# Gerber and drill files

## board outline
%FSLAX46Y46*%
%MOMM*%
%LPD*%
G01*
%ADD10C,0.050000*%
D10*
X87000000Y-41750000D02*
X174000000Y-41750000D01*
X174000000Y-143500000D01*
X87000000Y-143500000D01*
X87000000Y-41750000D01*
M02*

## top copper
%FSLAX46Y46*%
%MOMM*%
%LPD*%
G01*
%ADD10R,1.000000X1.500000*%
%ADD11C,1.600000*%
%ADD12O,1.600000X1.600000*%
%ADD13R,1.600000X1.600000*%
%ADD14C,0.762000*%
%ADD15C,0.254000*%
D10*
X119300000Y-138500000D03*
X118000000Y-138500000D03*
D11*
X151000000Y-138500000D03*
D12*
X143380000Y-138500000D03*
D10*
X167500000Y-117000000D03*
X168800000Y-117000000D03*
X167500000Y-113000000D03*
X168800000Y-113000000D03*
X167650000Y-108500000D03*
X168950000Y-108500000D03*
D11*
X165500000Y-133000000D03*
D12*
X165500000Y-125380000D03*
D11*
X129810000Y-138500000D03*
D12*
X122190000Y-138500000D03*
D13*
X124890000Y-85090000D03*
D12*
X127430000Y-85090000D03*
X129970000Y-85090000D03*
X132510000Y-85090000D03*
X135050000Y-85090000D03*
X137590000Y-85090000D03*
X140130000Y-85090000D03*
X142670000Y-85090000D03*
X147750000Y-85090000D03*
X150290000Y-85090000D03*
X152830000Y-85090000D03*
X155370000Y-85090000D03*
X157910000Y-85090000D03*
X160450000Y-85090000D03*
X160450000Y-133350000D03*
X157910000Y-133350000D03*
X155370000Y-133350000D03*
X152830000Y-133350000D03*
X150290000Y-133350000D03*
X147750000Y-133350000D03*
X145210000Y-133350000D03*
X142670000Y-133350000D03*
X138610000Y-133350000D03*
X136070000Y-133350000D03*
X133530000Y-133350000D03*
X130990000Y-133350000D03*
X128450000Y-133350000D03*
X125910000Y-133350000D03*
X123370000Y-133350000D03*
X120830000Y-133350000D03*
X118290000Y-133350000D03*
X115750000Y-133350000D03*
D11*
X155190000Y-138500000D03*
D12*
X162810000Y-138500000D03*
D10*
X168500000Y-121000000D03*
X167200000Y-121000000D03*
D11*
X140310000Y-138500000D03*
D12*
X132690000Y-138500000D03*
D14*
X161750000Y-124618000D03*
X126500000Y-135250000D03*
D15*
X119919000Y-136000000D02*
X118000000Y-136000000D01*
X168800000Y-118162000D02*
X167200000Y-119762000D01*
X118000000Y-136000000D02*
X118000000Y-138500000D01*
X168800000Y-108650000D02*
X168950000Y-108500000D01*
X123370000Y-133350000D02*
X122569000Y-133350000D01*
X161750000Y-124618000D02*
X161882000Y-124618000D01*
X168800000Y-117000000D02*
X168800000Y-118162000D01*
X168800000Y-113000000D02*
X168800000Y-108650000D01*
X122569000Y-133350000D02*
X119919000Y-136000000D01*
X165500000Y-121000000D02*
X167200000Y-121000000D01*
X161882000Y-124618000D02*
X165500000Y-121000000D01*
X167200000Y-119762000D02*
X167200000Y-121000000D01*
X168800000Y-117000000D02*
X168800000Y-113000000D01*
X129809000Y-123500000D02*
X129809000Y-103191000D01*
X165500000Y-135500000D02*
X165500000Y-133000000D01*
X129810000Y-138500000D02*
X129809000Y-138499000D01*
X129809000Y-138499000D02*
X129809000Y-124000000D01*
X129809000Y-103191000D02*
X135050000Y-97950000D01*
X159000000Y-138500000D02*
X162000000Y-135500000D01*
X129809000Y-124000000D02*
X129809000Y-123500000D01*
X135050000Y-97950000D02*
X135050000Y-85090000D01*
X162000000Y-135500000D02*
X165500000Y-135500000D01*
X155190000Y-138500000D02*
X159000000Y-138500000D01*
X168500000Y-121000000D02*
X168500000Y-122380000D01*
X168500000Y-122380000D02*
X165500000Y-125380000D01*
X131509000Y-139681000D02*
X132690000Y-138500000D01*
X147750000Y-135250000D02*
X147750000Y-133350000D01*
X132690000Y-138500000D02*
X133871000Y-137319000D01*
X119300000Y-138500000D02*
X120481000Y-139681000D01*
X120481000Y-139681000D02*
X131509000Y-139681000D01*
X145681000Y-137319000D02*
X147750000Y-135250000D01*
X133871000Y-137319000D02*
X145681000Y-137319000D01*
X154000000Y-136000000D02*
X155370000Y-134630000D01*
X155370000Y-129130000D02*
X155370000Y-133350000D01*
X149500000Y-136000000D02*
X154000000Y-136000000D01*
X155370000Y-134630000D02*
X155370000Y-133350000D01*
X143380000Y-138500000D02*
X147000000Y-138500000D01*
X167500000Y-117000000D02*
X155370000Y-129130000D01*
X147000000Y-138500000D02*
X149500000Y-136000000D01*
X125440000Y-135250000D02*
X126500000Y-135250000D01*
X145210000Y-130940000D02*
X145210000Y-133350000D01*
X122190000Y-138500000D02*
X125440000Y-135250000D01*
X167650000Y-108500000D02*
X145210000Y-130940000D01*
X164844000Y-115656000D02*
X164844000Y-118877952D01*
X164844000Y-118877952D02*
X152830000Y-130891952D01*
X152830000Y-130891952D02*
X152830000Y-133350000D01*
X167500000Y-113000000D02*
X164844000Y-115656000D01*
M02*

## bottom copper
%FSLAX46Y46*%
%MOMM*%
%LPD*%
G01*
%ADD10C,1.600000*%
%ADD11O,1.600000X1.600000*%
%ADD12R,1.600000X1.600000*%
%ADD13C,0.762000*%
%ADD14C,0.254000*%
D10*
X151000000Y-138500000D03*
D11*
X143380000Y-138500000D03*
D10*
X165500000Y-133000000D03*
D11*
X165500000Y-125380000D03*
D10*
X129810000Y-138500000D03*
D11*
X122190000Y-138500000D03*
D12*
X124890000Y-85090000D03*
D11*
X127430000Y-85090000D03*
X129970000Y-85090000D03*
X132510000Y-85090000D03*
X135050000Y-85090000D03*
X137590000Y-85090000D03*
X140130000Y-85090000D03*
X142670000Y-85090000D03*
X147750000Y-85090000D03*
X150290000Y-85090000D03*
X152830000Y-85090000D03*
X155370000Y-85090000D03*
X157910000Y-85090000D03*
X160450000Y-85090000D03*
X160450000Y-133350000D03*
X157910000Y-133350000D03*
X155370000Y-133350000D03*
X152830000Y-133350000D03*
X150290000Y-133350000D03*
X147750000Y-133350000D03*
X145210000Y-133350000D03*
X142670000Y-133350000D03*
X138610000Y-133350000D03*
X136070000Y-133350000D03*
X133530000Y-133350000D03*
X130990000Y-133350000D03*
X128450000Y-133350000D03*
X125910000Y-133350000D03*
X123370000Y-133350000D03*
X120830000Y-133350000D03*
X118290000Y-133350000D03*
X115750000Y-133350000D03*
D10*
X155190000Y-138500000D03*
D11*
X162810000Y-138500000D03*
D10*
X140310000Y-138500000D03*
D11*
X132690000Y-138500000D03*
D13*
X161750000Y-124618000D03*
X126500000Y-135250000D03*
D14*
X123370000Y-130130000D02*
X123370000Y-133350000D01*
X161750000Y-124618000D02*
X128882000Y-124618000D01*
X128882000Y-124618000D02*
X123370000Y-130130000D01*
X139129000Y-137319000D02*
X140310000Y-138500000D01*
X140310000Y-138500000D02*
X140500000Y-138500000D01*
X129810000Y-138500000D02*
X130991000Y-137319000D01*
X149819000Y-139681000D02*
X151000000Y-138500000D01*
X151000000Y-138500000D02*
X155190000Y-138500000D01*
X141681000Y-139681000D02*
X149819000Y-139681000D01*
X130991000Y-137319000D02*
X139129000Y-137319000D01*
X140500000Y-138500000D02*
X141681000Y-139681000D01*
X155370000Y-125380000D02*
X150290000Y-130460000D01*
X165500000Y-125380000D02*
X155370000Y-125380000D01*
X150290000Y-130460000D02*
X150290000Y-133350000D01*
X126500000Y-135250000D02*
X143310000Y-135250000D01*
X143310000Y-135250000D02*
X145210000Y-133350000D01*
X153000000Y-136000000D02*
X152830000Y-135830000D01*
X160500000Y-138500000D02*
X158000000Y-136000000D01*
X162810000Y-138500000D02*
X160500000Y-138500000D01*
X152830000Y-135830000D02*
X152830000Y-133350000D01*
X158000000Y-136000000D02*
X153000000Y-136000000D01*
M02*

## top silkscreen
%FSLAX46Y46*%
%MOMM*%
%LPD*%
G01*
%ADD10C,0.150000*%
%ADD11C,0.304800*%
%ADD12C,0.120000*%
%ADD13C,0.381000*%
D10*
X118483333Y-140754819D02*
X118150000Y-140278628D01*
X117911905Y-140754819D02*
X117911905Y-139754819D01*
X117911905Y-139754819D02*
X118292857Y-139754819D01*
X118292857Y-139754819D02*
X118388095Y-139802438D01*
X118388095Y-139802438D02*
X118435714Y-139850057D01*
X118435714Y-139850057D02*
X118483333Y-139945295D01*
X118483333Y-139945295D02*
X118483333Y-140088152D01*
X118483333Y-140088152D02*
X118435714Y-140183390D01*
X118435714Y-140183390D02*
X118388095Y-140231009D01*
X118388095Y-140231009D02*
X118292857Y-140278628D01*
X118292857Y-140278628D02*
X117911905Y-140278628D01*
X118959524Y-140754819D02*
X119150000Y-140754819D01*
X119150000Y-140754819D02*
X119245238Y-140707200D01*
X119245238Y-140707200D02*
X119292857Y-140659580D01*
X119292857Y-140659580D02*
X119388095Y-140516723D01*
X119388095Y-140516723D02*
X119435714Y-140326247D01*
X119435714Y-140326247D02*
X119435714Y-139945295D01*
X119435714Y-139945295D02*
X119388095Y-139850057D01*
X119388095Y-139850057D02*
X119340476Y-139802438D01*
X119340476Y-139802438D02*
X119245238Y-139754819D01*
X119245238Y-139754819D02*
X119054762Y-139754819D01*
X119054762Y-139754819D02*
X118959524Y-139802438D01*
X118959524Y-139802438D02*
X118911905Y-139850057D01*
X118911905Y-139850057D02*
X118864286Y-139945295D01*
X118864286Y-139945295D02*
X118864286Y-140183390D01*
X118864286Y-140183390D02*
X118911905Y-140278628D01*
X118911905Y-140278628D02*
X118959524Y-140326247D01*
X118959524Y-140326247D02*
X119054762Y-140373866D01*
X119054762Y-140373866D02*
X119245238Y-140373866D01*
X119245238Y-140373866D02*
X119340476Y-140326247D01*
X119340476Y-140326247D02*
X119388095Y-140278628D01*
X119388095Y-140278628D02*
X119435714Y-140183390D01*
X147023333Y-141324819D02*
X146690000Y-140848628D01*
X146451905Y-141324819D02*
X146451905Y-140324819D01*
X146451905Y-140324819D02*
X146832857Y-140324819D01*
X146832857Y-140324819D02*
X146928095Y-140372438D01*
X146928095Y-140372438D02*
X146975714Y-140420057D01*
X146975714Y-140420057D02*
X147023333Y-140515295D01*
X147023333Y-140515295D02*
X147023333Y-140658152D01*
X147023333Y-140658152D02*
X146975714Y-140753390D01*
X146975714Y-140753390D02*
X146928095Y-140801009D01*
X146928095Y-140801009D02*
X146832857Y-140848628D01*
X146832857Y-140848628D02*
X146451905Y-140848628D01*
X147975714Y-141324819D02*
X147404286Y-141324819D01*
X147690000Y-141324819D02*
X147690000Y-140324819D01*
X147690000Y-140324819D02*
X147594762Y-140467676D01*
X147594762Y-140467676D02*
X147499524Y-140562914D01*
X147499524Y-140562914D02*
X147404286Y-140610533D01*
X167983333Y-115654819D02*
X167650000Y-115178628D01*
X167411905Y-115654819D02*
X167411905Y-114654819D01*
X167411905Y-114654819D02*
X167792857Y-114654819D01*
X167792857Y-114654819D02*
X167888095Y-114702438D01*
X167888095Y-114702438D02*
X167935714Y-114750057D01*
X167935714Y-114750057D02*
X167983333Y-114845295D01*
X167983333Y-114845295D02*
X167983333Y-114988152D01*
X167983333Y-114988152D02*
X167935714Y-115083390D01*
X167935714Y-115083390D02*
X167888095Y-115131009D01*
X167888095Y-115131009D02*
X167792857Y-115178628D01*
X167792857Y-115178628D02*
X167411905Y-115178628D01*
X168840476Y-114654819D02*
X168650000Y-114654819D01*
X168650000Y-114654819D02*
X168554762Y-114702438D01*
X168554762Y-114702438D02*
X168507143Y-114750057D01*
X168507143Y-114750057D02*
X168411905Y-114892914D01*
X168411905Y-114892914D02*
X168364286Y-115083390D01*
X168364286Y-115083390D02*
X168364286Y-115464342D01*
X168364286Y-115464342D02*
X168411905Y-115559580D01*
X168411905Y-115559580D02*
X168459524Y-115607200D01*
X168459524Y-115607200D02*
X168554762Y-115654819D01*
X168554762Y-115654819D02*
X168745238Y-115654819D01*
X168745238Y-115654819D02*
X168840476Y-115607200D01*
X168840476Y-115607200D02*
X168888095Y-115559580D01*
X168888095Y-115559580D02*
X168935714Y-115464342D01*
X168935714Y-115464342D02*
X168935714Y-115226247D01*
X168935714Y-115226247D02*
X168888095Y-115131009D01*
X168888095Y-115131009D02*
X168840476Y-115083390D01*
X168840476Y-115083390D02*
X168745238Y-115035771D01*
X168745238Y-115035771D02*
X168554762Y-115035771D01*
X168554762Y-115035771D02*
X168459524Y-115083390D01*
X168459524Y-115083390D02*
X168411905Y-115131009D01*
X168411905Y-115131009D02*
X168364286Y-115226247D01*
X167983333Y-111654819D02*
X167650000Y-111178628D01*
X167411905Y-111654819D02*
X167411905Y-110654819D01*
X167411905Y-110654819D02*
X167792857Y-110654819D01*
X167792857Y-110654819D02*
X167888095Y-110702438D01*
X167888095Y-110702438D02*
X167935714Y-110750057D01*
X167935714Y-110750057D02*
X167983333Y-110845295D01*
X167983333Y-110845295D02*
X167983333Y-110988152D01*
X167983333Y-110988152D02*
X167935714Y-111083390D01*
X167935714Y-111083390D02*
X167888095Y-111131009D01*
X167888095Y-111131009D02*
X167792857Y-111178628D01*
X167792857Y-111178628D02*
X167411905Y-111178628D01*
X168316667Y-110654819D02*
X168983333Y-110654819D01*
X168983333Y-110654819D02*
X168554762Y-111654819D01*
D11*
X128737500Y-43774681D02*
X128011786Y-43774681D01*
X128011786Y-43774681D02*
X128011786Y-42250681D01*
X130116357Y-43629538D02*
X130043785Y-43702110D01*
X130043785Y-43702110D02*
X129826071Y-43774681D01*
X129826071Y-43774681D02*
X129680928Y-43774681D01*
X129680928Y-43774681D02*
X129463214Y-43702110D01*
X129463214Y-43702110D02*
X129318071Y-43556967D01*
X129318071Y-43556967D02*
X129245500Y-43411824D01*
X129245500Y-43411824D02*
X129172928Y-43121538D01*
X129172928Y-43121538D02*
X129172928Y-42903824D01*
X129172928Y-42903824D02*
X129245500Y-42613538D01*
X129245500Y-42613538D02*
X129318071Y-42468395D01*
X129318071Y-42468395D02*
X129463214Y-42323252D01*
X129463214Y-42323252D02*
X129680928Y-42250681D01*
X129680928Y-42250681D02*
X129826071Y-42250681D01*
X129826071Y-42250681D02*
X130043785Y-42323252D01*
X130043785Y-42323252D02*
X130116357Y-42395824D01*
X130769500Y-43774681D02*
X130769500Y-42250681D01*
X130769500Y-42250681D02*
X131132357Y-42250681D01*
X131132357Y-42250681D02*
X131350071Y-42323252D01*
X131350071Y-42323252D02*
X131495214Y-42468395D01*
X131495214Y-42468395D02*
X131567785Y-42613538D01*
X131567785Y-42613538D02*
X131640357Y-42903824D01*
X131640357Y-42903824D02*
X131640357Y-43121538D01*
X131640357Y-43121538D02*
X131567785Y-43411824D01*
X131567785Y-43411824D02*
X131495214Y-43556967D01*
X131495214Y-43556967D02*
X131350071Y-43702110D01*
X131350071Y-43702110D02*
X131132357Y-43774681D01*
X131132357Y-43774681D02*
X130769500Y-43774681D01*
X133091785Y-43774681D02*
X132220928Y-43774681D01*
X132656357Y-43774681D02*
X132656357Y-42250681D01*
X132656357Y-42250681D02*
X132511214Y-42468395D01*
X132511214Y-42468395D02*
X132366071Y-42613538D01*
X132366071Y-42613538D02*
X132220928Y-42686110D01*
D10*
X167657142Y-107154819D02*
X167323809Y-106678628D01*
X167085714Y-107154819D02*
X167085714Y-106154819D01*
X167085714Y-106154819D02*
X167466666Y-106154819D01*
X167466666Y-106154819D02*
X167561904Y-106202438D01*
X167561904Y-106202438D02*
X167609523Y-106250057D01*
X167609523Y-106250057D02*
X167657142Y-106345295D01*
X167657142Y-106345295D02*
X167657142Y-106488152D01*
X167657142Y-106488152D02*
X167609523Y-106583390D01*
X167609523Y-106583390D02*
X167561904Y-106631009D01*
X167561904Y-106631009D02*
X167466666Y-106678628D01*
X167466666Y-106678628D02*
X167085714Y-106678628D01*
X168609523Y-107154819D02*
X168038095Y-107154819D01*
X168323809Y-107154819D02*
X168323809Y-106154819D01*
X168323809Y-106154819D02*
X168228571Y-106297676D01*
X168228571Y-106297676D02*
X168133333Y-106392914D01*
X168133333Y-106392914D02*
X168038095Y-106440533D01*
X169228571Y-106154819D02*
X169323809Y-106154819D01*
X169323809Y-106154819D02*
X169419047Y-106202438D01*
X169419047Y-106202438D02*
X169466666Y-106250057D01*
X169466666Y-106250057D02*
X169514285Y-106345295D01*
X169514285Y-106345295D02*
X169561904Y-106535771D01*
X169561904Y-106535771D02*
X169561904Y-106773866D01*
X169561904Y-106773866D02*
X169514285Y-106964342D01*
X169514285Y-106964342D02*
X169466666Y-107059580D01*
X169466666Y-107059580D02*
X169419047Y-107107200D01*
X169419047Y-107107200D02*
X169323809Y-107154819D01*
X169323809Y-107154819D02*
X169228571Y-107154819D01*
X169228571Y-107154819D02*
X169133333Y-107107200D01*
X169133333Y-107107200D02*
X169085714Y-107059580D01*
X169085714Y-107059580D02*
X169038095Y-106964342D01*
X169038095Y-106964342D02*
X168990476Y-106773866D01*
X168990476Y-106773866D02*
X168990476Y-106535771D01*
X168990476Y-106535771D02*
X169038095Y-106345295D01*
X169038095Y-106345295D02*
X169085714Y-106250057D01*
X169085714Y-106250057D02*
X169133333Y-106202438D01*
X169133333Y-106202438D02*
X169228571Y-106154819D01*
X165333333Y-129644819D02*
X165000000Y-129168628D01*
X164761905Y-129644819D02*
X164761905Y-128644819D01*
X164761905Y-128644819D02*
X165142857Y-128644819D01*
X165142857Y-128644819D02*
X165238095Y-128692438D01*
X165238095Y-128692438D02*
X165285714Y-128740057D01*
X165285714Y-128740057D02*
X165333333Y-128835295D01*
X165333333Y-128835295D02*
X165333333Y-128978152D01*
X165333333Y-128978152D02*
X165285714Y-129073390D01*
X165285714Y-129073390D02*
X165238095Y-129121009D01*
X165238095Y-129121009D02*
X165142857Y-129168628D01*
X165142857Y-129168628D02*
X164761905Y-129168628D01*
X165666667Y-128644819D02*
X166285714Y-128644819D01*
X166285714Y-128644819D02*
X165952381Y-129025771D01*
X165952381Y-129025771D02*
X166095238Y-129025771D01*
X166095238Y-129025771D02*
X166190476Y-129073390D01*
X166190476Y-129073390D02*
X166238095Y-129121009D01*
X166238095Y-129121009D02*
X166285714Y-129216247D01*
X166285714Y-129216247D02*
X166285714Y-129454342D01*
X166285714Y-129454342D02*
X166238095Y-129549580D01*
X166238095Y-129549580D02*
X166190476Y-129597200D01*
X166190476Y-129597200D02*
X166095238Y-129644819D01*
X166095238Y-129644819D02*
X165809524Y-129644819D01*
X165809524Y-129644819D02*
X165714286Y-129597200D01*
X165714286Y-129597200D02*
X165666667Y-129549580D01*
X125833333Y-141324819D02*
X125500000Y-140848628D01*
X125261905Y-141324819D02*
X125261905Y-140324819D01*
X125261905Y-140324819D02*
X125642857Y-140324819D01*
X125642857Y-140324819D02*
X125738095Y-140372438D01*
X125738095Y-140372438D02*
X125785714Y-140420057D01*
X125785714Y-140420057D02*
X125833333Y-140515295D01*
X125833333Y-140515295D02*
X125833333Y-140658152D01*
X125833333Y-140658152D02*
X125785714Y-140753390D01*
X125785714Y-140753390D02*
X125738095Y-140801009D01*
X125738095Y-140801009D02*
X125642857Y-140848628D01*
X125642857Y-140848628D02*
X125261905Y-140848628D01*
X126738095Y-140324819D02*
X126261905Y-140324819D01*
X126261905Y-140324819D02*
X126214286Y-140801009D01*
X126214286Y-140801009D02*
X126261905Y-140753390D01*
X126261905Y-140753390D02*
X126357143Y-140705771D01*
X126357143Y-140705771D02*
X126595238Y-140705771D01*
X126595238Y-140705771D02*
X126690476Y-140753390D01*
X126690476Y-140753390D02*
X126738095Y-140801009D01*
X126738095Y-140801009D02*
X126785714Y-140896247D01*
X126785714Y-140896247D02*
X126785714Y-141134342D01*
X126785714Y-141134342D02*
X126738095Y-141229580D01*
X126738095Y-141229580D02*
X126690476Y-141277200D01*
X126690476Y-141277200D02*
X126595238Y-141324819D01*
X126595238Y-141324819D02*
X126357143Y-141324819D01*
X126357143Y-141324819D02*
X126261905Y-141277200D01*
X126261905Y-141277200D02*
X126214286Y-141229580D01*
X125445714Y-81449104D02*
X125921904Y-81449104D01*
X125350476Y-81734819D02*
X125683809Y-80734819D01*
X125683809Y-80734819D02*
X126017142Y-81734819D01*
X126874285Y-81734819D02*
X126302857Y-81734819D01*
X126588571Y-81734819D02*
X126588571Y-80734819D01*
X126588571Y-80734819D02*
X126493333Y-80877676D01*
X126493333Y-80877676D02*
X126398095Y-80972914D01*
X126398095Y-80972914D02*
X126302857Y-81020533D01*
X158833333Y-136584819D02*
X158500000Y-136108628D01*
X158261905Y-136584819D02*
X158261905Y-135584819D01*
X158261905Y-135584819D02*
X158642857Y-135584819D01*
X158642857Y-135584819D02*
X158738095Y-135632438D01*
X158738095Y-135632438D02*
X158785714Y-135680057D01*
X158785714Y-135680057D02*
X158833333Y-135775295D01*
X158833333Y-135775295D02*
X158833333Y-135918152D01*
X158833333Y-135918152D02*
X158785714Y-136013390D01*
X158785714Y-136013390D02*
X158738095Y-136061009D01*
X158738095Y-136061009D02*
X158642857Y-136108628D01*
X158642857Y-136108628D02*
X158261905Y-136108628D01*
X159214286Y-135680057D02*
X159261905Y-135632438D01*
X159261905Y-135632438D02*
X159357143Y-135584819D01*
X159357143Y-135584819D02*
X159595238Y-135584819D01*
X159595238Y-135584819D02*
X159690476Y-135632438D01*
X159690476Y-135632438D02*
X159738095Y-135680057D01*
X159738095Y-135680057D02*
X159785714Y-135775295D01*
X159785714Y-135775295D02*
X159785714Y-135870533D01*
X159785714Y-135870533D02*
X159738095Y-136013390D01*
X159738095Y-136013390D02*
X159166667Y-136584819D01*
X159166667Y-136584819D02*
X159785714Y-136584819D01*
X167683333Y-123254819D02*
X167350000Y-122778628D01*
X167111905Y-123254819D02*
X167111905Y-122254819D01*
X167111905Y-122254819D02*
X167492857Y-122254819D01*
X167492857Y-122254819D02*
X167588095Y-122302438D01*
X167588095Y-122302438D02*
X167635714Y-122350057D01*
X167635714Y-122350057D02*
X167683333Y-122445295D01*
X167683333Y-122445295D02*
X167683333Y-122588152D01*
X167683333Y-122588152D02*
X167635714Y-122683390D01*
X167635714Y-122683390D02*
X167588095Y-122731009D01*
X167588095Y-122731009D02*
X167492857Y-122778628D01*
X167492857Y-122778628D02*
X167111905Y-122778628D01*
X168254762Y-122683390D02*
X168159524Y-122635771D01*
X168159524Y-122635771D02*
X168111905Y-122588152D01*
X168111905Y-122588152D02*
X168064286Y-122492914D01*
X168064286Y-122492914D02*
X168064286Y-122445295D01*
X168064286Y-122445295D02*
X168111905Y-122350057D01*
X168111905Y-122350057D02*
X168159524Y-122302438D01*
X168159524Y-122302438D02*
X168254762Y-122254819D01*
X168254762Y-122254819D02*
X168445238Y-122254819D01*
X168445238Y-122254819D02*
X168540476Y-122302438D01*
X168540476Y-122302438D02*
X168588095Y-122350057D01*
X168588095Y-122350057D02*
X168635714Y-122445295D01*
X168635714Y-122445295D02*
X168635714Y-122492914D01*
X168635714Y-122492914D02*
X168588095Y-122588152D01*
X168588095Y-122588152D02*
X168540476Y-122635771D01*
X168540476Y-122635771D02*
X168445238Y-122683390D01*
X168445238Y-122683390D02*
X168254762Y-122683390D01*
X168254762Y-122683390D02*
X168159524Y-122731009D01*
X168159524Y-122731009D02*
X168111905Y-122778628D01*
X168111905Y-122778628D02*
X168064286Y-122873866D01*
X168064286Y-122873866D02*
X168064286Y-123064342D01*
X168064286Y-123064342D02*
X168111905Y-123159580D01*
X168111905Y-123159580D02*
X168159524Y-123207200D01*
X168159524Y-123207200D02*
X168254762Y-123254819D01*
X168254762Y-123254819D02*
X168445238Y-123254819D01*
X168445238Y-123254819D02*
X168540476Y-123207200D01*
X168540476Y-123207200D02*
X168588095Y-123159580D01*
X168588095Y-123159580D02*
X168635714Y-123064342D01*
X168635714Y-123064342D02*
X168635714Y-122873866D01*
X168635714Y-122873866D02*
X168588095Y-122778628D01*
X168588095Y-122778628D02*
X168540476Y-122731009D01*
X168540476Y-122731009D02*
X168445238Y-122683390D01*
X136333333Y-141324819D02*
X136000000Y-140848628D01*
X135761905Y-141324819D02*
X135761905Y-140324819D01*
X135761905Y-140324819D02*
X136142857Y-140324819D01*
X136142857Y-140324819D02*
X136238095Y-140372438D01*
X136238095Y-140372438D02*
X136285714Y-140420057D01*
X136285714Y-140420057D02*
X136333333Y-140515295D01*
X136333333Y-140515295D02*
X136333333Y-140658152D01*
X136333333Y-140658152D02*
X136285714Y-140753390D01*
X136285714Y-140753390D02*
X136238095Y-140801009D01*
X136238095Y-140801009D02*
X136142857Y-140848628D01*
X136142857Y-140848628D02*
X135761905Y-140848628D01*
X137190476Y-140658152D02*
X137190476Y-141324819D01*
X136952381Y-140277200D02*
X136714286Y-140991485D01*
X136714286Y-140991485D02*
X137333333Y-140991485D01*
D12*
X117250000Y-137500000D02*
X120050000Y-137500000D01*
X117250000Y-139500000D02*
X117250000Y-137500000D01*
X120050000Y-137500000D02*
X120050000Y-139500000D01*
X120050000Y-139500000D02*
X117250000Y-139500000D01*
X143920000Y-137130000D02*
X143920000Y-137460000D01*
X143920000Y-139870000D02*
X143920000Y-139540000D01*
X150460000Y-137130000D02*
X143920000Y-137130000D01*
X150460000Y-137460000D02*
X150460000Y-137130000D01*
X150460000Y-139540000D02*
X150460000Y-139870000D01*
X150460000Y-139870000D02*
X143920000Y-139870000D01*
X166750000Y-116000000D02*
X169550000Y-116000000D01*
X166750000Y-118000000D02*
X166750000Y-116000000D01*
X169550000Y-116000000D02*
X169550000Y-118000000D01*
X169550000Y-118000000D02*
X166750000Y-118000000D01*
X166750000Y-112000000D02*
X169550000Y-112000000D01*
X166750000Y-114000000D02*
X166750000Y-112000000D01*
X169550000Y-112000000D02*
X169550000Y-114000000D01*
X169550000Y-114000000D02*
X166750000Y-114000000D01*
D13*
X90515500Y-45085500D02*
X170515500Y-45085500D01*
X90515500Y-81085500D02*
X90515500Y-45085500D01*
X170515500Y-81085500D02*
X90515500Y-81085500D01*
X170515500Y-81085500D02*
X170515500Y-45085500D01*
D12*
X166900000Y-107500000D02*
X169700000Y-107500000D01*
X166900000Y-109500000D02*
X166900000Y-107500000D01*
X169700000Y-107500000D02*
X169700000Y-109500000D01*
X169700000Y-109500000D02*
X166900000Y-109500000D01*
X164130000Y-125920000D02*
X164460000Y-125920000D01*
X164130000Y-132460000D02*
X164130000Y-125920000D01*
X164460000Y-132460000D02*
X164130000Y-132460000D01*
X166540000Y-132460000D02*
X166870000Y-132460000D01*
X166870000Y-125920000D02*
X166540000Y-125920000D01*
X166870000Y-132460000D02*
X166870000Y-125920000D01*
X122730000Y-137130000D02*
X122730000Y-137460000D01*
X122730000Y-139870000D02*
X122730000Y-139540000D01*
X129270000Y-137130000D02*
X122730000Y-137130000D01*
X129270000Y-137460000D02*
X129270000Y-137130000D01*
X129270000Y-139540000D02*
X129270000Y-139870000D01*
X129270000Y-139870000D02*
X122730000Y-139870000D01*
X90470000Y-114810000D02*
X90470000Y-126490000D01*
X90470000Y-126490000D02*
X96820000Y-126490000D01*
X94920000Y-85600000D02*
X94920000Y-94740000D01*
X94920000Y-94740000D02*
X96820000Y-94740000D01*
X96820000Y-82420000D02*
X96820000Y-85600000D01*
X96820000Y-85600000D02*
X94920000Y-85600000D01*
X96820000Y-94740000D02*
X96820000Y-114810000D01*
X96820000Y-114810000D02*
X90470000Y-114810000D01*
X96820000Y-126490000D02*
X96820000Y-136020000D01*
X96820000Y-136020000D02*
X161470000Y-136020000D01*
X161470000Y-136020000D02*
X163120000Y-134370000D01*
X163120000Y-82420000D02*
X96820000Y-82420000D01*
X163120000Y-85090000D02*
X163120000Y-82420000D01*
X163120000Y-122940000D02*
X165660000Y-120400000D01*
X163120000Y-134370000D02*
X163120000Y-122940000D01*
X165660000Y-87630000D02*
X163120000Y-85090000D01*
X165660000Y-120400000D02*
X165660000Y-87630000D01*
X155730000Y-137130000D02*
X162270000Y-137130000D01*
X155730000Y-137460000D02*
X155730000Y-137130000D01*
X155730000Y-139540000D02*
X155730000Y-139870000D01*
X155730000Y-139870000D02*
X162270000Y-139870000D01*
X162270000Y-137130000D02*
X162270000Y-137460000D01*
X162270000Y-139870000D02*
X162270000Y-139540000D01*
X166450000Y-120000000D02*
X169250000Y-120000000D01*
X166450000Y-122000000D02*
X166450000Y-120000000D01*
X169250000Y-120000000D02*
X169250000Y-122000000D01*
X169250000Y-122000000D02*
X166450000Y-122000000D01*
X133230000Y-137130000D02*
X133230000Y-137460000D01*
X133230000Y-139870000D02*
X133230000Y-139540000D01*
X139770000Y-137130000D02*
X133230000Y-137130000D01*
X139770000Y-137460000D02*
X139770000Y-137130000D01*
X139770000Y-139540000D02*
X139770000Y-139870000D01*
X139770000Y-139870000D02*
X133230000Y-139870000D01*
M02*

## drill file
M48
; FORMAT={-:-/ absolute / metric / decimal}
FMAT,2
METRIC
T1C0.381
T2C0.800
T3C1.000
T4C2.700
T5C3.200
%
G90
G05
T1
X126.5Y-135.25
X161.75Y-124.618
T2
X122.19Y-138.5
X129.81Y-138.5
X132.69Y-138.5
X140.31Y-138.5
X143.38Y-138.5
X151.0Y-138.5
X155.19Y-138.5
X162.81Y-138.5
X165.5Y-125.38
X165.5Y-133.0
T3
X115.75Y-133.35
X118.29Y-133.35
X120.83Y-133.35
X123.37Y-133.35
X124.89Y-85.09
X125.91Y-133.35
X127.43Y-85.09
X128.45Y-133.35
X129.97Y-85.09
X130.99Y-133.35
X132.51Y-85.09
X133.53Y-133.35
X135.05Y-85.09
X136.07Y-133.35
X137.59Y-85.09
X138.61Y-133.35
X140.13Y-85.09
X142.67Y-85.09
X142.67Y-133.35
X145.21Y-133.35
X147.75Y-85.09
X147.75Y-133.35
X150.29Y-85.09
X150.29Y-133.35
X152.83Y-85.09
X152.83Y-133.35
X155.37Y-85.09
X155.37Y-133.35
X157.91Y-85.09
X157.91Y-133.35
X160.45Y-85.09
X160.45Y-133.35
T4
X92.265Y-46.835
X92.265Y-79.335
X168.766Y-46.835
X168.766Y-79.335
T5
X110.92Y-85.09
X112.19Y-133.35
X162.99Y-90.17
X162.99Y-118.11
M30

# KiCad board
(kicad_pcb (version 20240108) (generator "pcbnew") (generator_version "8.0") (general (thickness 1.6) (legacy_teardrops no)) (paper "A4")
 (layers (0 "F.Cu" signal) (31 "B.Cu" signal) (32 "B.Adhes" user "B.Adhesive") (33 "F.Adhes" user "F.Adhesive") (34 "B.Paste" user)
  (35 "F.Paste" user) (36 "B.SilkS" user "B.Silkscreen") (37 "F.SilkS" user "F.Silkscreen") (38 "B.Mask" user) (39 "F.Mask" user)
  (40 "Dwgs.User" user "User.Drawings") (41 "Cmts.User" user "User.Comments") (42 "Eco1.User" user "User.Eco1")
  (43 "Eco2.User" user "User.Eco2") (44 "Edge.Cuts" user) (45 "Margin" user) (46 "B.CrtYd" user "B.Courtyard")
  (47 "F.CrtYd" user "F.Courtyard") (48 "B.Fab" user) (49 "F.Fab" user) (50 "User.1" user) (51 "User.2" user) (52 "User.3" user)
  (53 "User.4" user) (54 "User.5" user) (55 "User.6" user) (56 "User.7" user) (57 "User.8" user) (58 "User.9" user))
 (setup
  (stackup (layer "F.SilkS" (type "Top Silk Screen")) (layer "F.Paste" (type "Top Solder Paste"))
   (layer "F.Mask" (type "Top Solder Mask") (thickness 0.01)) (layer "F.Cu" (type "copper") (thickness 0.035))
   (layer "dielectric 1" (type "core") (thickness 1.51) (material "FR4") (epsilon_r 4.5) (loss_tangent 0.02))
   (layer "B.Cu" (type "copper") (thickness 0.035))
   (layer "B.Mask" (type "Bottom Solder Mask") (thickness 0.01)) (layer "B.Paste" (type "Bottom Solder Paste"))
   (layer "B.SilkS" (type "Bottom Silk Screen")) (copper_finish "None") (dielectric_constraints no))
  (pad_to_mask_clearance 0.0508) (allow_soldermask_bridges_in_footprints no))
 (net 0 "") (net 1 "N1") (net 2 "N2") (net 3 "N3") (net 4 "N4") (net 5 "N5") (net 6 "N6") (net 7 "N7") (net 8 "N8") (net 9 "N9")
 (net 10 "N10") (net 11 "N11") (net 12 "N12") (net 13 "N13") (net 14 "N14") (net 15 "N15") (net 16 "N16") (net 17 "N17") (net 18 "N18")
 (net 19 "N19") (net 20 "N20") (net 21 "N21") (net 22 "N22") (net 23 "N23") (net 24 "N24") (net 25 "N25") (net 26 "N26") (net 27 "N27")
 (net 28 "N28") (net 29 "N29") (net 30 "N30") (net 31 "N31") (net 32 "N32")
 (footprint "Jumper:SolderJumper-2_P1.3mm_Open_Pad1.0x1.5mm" (layer "F.Cu") (at 118.65 138.5 180)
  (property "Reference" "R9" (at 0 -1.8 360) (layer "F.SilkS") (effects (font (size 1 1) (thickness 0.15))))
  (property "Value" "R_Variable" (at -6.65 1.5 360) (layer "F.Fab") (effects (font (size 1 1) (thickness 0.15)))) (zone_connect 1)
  (fp_line (start 1.4 1) (end -1.4 1) (stroke (width 0.12) (type solid)) (layer "F.SilkS"))
  (fp_line (start 1.4 -1) (end 1.4 1) (stroke (width 0.12) (type solid)) (layer "F.SilkS"))
  (fp_line (start -1.4 1) (end -1.4 -1) (stroke (width 0.12) (type solid)) (layer "F.SilkS"))
  (fp_line (start -1.4 -1) (end 1.4 -1) (stroke (width 0.12) (type solid)) (layer "F.SilkS"))
  (pad "1" smd rect (at -0.65 0 180) (size 1 1.5) (layers "F.Cu" "F.Mask") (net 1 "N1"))
  (pad "2" smd rect (at 0.65 0 180) (size 1 1.5) (layers "F.Cu" "F.Mask") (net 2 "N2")))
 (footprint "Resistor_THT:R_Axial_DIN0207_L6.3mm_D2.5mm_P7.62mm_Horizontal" (layer "F.Cu") (at 151 138.5 180)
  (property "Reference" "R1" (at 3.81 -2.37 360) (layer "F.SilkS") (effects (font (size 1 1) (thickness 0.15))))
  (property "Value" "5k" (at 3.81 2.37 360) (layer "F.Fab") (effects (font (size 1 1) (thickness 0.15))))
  (fp_line (start 7.08 1.37) (end 7.08 1.04) (stroke (width 0.12) (type solid)) (layer "F.SilkS"))
  (fp_line (start 7.08 -1.37) (end 7.08 -1.04) (stroke (width 0.12) (type solid)) (layer "F.SilkS"))
  (fp_line (start 0.54 1.37) (end 7.08 1.37) (stroke (width 0.12) (type solid)) (layer "F.SilkS"))
  (fp_line (start 0.54 1.04) (end 0.54 1.37) (stroke (width 0.12) (type solid)) (layer "F.SilkS"))
  (fp_line (start 0.54 -1.04) (end 0.54 -1.37) (stroke (width 0.12) (type solid)) (layer "F.SilkS"))
  (fp_line (start 0.54 -1.37) (end 7.08 -1.37) (stroke (width 0.12) (type solid)) (layer "F.SilkS"))
  (pad "1" thru_hole circle (at 0 0 180) (size 1.6 1.6) (drill 0.8) (layers "*.Cu" "*.Mask") (remove_unused_layers no) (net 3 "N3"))
  (pad "2" thru_hole oval (at 7.62 0 180) (size 1.6 1.6) (drill 0.8) (layers "*.Cu" "*.Mask") (remove_unused_layers no) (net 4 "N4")))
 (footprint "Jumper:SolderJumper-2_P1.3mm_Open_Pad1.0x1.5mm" (layer "F.Cu") (at 168.15 117)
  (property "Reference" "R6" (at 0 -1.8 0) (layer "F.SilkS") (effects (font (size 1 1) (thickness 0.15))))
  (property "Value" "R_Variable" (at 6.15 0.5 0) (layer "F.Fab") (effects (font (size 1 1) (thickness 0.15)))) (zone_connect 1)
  (fp_line (start -1.4 -1) (end 1.4 -1) (stroke (width 0.12) (type solid)) (layer "F.SilkS"))
  (fp_line (start -1.4 1) (end -1.4 -1) (stroke (width 0.12) (type solid)) (layer "F.SilkS"))
  (fp_line (start 1.4 -1) (end 1.4 1) (stroke (width 0.12) (type solid)) (layer "F.SilkS"))
  (fp_line (start 1.4 1) (end -1.4 1) (stroke (width 0.12) (type solid)) (layer "F.SilkS"))
  (pad "1" smd rect (at -0.65 0) (size 1 1.5) (layers "F.Cu" "F.Mask") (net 4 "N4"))
  (pad "2" smd rect (at 0.65 0) (size 1 1.5) (layers "F.Cu" "F.Mask") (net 2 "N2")))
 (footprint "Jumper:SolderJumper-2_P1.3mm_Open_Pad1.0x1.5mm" (layer "F.Cu") (at 168.15 113)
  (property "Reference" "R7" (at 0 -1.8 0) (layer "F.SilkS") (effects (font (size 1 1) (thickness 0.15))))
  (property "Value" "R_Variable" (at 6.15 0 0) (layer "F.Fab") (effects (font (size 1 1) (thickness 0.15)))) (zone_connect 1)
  (fp_line (start -1.4 -1) (end 1.4 -1) (stroke (width 0.12) (type solid)) (layer "F.SilkS"))
  (fp_line (start -1.4 1) (end -1.4 -1) (stroke (width 0.12) (type solid)) (layer "F.SilkS"))
  (fp_line (start 1.4 -1) (end 1.4 1) (stroke (width 0.12) (type solid)) (layer "F.SilkS"))
  (fp_line (start 1.4 1) (end -1.4 1) (stroke (width 0.12) (type solid)) (layer "F.SilkS"))
  (pad "1" smd rect (at -0.65 0) (size 1 1.5) (layers "F.Cu" "F.Mask") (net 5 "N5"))
  (pad "2" smd rect (at 0.65 0) (size 1 1.5) (layers "F.Cu" "F.Mask") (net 2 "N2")))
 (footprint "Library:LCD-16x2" (layer "F.Cu") (at 130.5155 63.0855)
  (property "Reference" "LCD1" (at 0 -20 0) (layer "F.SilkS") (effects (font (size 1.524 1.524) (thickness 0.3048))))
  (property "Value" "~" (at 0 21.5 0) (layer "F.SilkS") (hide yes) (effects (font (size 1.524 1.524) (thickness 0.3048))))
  (fp_line (start -40 -18) (end 40 -18) (stroke (width 0.381) (type solid)) (layer "F.SilkS"))
  (fp_line (start -40 18) (end -40 -18) (stroke (width 0.381) (type solid)) (layer "F.SilkS"))
  (fp_line (start 40 18) (end -40 18) (stroke (width 0.381) (type solid)) (layer "F.SilkS"))
  (fp_line (start 40 18) (end 40 -18) (stroke (width 0.381) (type solid)) (layer "F.SilkS"))
  (pad "" np_thru_hole circle (at -38.25 -16.25) (size 0.01 0.01) (drill 2.7) (layers "F&B.Cu" "*.Mask"))
  (pad "" np_thru_hole circle (at -38.25 16.25 90) (size 0.01 0.01) (drill 2.7) (layers "F&B.Cu" "*.Mask"))
  (pad "" np_thru_hole circle (at 38.25 -16.25) (size 0.01 0.01) (drill 2.7) (layers "F&B.Cu" "*.Mask"))
  (pad "" np_thru_hole circle (at 38.25 16.25) (size 0.01 0.01) (drill 2.7) (layers "F&B.Cu" "*.Mask")))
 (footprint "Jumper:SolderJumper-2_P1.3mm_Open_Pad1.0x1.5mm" (layer "F.Cu") (at 168.3 108.5)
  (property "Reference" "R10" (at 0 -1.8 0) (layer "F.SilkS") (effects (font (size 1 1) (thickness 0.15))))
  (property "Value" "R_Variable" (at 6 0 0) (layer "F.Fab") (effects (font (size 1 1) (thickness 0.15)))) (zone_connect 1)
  (fp_line (start -1.4 -1) (end 1.4 -1) (stroke (width 0.12) (type solid)) (layer "F.SilkS"))
  (fp_line (start -1.4 1) (end -1.4 -1) (stroke (width 0.12) (type solid)) (layer "F.SilkS"))
  (fp_line (start 1.4 -1) (end 1.4 1) (stroke (width 0.12) (type solid)) (layer "F.SilkS"))
  (fp_line (start 1.4 1) (end -1.4 1) (stroke (width 0.12) (type solid)) (layer "F.SilkS"))
  (pad "1" smd rect (at -0.65 0) (size 1 1.5) (layers "F.Cu" "F.Mask") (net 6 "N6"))
  (pad "2" smd rect (at 0.65 0) (size 1 1.5) (layers "F.Cu" "F.Mask") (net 2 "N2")))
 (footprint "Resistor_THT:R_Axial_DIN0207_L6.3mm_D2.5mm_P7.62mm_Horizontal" (layer "F.Cu") (at 165.5 133 90)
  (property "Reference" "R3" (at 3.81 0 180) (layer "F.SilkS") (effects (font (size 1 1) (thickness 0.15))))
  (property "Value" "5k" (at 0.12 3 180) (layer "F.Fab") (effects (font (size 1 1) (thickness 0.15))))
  (fp_line (start 7.08 -1.37) (end 7.08 -1.04) (stroke (width 0.12) (type solid)) (layer "F.SilkS"))
  (fp_line (start 0.54 -1.37) (end 7.08 -1.37) (stroke (width 0.12) (type solid)) (layer "F.SilkS"))
  (fp_line (start 0.54 -1.04) (end 0.54 -1.37) (stroke (width 0.12) (type solid)) (layer "F.SilkS"))
  (fp_line (start 0.54 1.04) (end 0.54 1.37) (stroke (width 0.12) (type solid)) (layer "F.SilkS"))
  (fp_line (start 7.08 1.37) (end 7.08 1.04) (stroke (width 0.12) (type solid)) (layer "F.SilkS"))
  (fp_line (start 0.54 1.37) (end 7.08 1.37) (stroke (width 0.12) (type solid)) (layer "F.SilkS"))
  (pad "1" thru_hole circle (at 0 0 90) (size 1.6 1.6) (drill 0.8) (layers "*.Cu" "*.Mask") (remove_unused_layers no) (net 3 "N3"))
  (pad "2" thru_hole oval (at 7.62 0 90) (size 1.6 1.6) (drill 0.8) (layers "*.Cu" "*.Mask") (remove_unused_layers no) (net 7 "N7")))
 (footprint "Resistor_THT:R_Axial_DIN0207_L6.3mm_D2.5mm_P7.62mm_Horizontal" (layer "F.Cu") (at 129.81 138.5 180)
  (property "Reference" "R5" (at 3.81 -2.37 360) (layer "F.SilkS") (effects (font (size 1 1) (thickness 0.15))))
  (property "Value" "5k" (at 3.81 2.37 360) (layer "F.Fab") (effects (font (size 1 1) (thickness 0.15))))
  (fp_line (start 7.08 1.37) (end 7.08 1.04) (stroke (width 0.12) (type solid)) (layer "F.SilkS"))
  (fp_line (start 7.08 -1.37) (end 7.08 -1.04) (stroke (width 0.12) (type solid)) (layer "F.SilkS"))
  (fp_line (start 0.54 1.37) (end 7.08 1.37) (stroke (width 0.12) (type solid)) (layer "F.SilkS"))
  (fp_line (start 0.54 1.04) (end 0.54 1.37) (stroke (width 0.12) (type solid)) (layer "F.SilkS"))
  (fp_line (start 0.54 -1.04) (end 0.54 -1.37) (stroke (width 0.12) (type solid)) (layer "F.SilkS"))
  (fp_line (start 0.54 -1.37) (end 7.08 -1.37) (stroke (width 0.12) (type solid)) (layer "F.SilkS"))
  (pad "1" thru_hole circle (at 0 0 180) (size 1.6 1.6) (drill 0.8) (layers "*.Cu" "*.Mask") (remove_unused_layers no) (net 3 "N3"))
  (pad "2" thru_hole oval (at 7.62 0 180) (size 1.6 1.6) (drill 0.8) (layers "*.Cu" "*.Mask") (remove_unused_layers no) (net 6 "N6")))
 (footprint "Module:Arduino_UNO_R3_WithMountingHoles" (layer "F.Cu") (at 124.89 85.09)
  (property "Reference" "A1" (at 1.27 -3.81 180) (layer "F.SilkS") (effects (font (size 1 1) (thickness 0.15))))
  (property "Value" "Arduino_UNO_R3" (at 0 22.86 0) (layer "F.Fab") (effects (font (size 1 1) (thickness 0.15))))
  (fp_line (start -34.42 29.72) (end -34.42 41.4) (stroke (width 0.12) (type solid)) (layer "F.SilkS"))
  (fp_line (start -34.42 41.4) (end -28.07 41.4) (stroke (width 0.12) (type solid)) (layer "F.SilkS"))
  (fp_line (start -29.97 0.51) (end -29.97 9.65) (stroke (width 0.12) (type solid)) (layer "F.SilkS"))
  (fp_line (start -29.97 9.65) (end -28.07 9.65) (stroke (width 0.12) (type solid)) (layer "F.SilkS"))
  (fp_line (start -28.07 -2.67) (end -28.07 0.51) (stroke (width 0.12) (type solid)) (layer "F.SilkS"))
  (fp_line (start -28.07 0.51) (end -29.97 0.51) (stroke (width 0.12) (type solid)) (layer "F.SilkS"))
  (fp_line (start -28.07 9.65) (end -28.07 29.72) (stroke (width 0.12) (type solid)) (layer "F.SilkS"))
  (fp_line (start -28.07 29.72) (end -34.42 29.72) (stroke (width 0.12) (type solid)) (layer "F.SilkS"))
  (fp_line (start -28.07 41.4) (end -28.07 50.93) (stroke (width 0.12) (type solid)) (layer "F.SilkS"))
  (fp_line (start -28.07 50.93) (end 36.58 50.93) (stroke (width 0.12) (type solid)) (layer "F.SilkS"))
  (fp_line (start 36.58 50.93) (end 38.23 49.28) (stroke (width 0.12) (type solid)) (layer "F.SilkS"))
  (fp_line (start 38.23 -2.67) (end -28.07 -2.67) (stroke (width 0.12) (type solid)) (layer "F.SilkS"))
  (fp_line (start 38.23 0) (end 38.23 -2.67) (stroke (width 0.12) (type solid)) (layer "F.SilkS"))
  (fp_line (start 38.23 37.85) (end 40.77 35.31) (stroke (width 0.12) (type solid)) (layer "F.SilkS"))
  (fp_line (start 38.23 49.28) (end 38.23 37.85) (stroke (width 0.12) (type solid)) (layer "F.SilkS"))
  (fp_line (start 40.77 2.54) (end 38.23 0) (stroke (width 0.12) (type solid)) (layer "F.SilkS"))
  (fp_line (start 40.77 35.31) (end 40.77 2.54) (stroke (width 0.12) (type solid)) (layer "F.SilkS"))
  (pad "" np_thru_hole circle (at -13.97 0 90) (size 3.2 3.2) (drill 3.2) (layers "*.Cu" "*.Mask"))
  (pad "" np_thru_hole circle (at -12.7 48.26 90) (size 3.2 3.2) (drill 3.2) (layers "*.Cu" "*.Mask"))
  (pad "" np_thru_hole circle (at 38.1 5.08 90) (size 3.2 3.2) (drill 3.2) (layers "*.Cu" "*.Mask"))
  (pad "" np_thru_hole circle (at 38.1 33.02 90) (size 3.2 3.2) (drill 3.2) (layers "*.Cu" "*.Mask"))
  (pad "1" thru_hole rect (at 0 0 90) (size 1.6 1.6) (drill 1) (layers "*.Cu" "*.Mask") (remove_unused_layers no) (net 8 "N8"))
  (pad "2" thru_hole oval (at 2.54 0 90) (size 1.6 1.6) (drill 1) (layers "*.Cu" "*.Mask") (remove_unused_layers no) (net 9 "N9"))
  (pad "3" thru_hole oval (at 5.08 0 90) (size 1.6 1.6) (drill 1) (layers "*.Cu" "*.Mask") (remove_unused_layers no) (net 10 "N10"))
  (pad "4" thru_hole oval (at 7.62 0 90) (size 1.6 1.6) (drill 1) (layers "*.Cu" "*.Mask") (remove_unused_layers no) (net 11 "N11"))
  (pad "5" thru_hole oval (at 10.16 0 90) (size 1.6 1.6) (drill 1) (layers "*.Cu" "*.Mask") (remove_unused_layers no) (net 3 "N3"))
  (pad "6" thru_hole oval (at 12.7 0 90) (size 1.6 1.6) (drill 1) (layers "*.Cu" "*.Mask") (remove_unused_layers no) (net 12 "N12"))
  (pad "7" thru_hole oval (at 15.24 0 90) (size 1.6 1.6) (drill 1) (layers "*.Cu" "*.Mask") (remove_unused_layers no) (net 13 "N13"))
  (pad "8" thru_hole oval (at 17.78 0 90) (size 1.6 1.6) (drill 1) (layers "*.Cu" "*.Mask") (remove_unused_layers no) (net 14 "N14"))
  (pad "9" thru_hole oval (at 22.86 0 90) (size 1.6 1.6) (drill 1) (layers "*.Cu" "*.Mask") (remove_unused_layers no) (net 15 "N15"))
  (pad "10" thru_hole oval (at 25.4 0 90) (size 1.6 1.6) (drill 1) (layers "*.Cu" "*.Mask") (remove_unused_layers no) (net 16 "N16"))
  (pad "11" thru_hole oval (at 27.94 0 90) (size 1.6 1.6) (drill 1) (layers "*.Cu" "*.Mask") (remove_unused_layers no) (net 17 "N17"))
  (pad "12" thru_hole oval (at 30.48 0 90) (size 1.6 1.6) (drill 1) (layers "*.Cu" "*.Mask") (remove_unused_layers no) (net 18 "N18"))
  (pad "13" thru_hole oval (at 33.02 0 90) (size 1.6 1.6) (drill 1) (layers "*.Cu" "*.Mask") (remove_unused_layers no) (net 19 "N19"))
  (pad "14" thru_hole oval (at 35.56 0 90) (size 1.6 1.6) (drill 1) (layers "*.Cu" "*.Mask") (remove_unused_layers no) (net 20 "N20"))
  (pad "15" thru_hole oval (at 35.56 48.26 90) (size 1.6 1.6) (drill 1) (layers "*.Cu" "*.Mask") (remove_unused_layers no) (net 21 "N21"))
  (pad "16" thru_hole oval (at 33.02 48.26 90) (size 1.6 1.6) (drill 1) (layers "*.Cu" "*.Mask") (remove_unused_layers no) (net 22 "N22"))
  (pad "17" thru_hole oval (at 30.48 48.26 90) (size 1.6 1.6) (drill 1) (layers "*.Cu" "*.Mask") (remove_unused_layers no) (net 4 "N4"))
  (pad "18" thru_hole oval (at 27.94 48.26 90) (size 1.6 1.6) (drill 1) (layers "*.Cu" "*.Mask") (remove_unused_layers no) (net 5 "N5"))
  (pad "19" thru_hole oval (at 25.4 48.26 90) (size 1.6 1.6) (drill 1) (layers "*.Cu" "*.Mask") (remove_unused_layers no) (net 7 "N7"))
  (pad "20" thru_hole oval (at 22.86 48.26 90) (size 1.6 1.6) (drill 1) (layers "*.Cu" "*.Mask") (remove_unused_layers no) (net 1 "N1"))
  (pad "21" thru_hole oval (at 20.32 48.26 90) (size 1.6 1.6) (drill 1) (layers "*.Cu" "*.Mask") (remove_unused_layers no) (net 6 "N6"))
  (pad "22" thru_hole oval (at 17.78 48.26 90) (size 1.6 1.6) (drill 1) (layers "*.Cu" "*.Mask") (remove_unused_layers no) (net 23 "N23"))
  (pad "23" thru_hole oval (at 13.72 48.26 90) (size 1.6 1.6) (drill 1) (layers "*.Cu" "*.Mask") (remove_unused_layers no) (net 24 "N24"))
  (pad "24" thru_hole oval (at 11.18 48.26 90) (size 1.6 1.6) (drill 1) (layers "*.Cu" "*.Mask") (remove_unused_layers no) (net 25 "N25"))
  (pad "25" thru_hole oval (at 8.64 48.26 90) (size 1.6 1.6) (drill 1) (layers "*.Cu" "*.Mask") (remove_unused_layers no) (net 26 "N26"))
  (pad "26" thru_hole oval (at 6.1 48.26 90) (size 1.6 1.6) (drill 1) (layers "*.Cu" "*.Mask") (remove_unused_layers no) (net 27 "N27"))
  (pad "27" thru_hole oval (at 3.56 48.26 90) (size 1.6 1.6) (drill 1) (layers "*.Cu" "*.Mask") (remove_unused_layers no) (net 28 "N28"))
  (pad "28" thru_hole oval (at 1.02 48.26 90) (size 1.6 1.6) (drill 1) (layers "*.Cu" "*.Mask") (remove_unused_layers no) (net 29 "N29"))
  (pad "29" thru_hole oval (at -1.52 48.26 90) (size 1.6 1.6) (drill 1) (layers "*.Cu" "*.Mask") (remove_unused_layers no) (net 2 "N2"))
  (pad "30" thru_hole oval (at -4.06 48.26 90) (size 1.6 1.6) (drill 1) (layers "*.Cu" "*.Mask") (remove_unused_layers no) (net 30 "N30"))
  (pad "31" thru_hole oval (at -6.6 48.26 90) (size 1.6 1.6) (drill 1) (layers "*.Cu" "*.Mask") (remove_unused_layers no) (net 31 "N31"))
  (pad "32" thru_hole oval (at -9.14 48.26 90) (size 1.6 1.6) (drill 1) (layers "*.Cu" "*.Mask") (remove_unused_layers no) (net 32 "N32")))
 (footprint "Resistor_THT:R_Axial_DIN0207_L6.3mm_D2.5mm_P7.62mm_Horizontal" (layer "F.Cu") (at 155.19 138.5)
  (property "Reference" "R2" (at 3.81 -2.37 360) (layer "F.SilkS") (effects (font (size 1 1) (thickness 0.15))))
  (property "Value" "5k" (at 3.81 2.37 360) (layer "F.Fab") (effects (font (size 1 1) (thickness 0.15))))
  (fp_line (start 0.54 -1.37) (end 7.08 -1.37) (stroke (width 0.12) (type solid)) (layer "F.SilkS"))
  (fp_line (start 0.54 -1.04) (end 0.54 -1.37) (stroke (width 0.12) (type solid)) (layer "F.SilkS"))
  (fp_line (start 0.54 1.04) (end 0.54 1.37) (stroke (width 0.12) (type solid)) (layer "F.SilkS"))
  (fp_line (start 0.54 1.37) (end 7.08 1.37) (stroke (width 0.12) (type solid)) (layer "F.SilkS"))
  (fp_line (start 7.08 -1.37) (end 7.08 -1.04) (stroke (width 0.12) (type solid)) (layer "F.SilkS"))
  (fp_line (start 7.08 1.37) (end 7.08 1.04) (stroke (width 0.12) (type solid)) (layer "F.SilkS"))
  (pad "1" thru_hole circle (at 0 0) (size 1.6 1.6) (drill 0.8) (layers "*.Cu" "*.Mask") (remove_unused_layers no) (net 3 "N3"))
  (pad "2" thru_hole oval (at 7.62 0) (size 1.6 1.6) (drill 0.8) (layers "*.Cu" "*.Mask") (remove_unused_layers no) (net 5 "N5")))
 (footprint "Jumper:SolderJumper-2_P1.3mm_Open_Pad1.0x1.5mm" (layer "F.Cu") (at 167.85 121 180)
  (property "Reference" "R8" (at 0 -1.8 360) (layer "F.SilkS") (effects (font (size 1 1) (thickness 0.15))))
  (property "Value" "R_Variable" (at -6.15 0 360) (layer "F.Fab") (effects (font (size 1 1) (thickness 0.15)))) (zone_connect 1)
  (fp_line (start 1.4 1) (end -1.4 1) (stroke (width 0.12) (type solid)) (layer "F.SilkS"))
  (fp_line (start 1.4 -1) (end 1.4 1) (stroke (width 0.12) (type solid)) (layer "F.SilkS"))
  (fp_line (start -1.4 1) (end -1.4 -1) (stroke (width 0.12) (type solid)) (layer "F.SilkS"))
  (fp_line (start -1.4 -1) (end 1.4 -1) (stroke (width 0.12) (type solid)) (layer "F.SilkS"))
  (pad "1" smd rect (at -0.65 0 180) (size 1 1.5) (layers "F.Cu" "F.Mask") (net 7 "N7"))
  (pad "2" smd rect (at 0.65 0 180) (size 1 1.5) (layers "F.Cu" "F.Mask") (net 2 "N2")))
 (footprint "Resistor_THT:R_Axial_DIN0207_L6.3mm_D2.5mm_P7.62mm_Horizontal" (layer "F.Cu") (at 140.31 138.5 180)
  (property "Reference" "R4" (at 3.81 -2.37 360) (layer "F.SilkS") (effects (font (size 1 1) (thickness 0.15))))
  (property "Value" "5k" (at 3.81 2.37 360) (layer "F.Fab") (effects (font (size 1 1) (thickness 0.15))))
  (fp_line (start 7.08 1.37) (end 7.08 1.04) (stroke (width 0.12) (type solid)) (layer "F.SilkS"))
  (fp_line (start 7.08 -1.37) (end 7.08 -1.04) (stroke (width 0.12) (type solid)) (layer "F.SilkS"))
  (fp_line (start 0.54 1.37) (end 7.08 1.37) (stroke (width 0.12) (type solid)) (layer "F.SilkS"))
  (fp_line (start 0.54 1.04) (end 0.54 1.37) (stroke (width 0.12) (type solid)) (layer "F.SilkS"))
  (fp_line (start 0.54 -1.04) (end 0.54 -1.37) (stroke (width 0.12) (type solid)) (layer "F.SilkS"))
  (fp_line (start 0.54 -1.37) (end 7.08 -1.37) (stroke (width 0.12) (type solid)) (layer "F.SilkS"))
  (pad "1" thru_hole circle (at 0 0 180) (size 1.6 1.6) (drill 0.8) (layers "*.Cu" "*.Mask") (remove_unused_layers no) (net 3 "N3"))
  (pad "2" thru_hole oval (at 7.62 0 180) (size 1.6 1.6) (drill 0.8) (layers "*.Cu" "*.Mask") (remove_unused_layers no) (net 1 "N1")))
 (gr_rect (start 87 41.75) (end 174 143.5) (stroke (width 0.05) (type default)) (fill none) (layer "Edge.Cuts"))
 (segment (start 119.919 136) (end 118 136) (width 0.254) (layer "F.Cu") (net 2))
 (segment (start 168.8 118.162) (end 167.2 119.762) (width 0.254) (layer "F.Cu") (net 2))
 (segment (start 118 136) (end 118 138.5) (width 0.254) (layer "F.Cu") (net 2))
 (segment (start 168.8 108.65) (end 168.95 108.5) (width 0.254) (layer "F.Cu") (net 2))
 (segment (start 123.37 133.35) (end 122.569 133.35) (width 0.254) (layer "F.Cu") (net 2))
 (segment (start 161.75 124.618) (end 161.882 124.618) (width 0.254) (layer "F.Cu") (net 2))
 (segment (start 168.8 117) (end 168.8 118.162) (width 0.254) (layer "F.Cu") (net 2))
 (segment (start 168.8 113) (end 168.8 108.65) (width 0.254) (layer "F.Cu") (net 2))
 (segment (start 122.569 133.35) (end 119.919 136) (width 0.254) (layer "F.Cu") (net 2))
 (segment (start 165.5 121) (end 167.2 121) (width 0.254) (layer "F.Cu") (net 2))
 (segment (start 161.882 124.618) (end 165.5 121) (width 0.254) (layer "F.Cu") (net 2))
 (segment (start 167.2 119.762) (end 167.2 121) (width 0.254) (layer "F.Cu") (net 2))
 (segment (start 168.8 117) (end 168.8 113) (width 0.254) (layer "F.Cu") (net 2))
 (via (at 161.75 124.618) (size 0.762) (drill 0.381) (layers "F.Cu" "B.Cu") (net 2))
 (segment (start 123.37 130.13) (end 123.37 133.35) (width 0.254) (layer "B.Cu") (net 2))
 (segment (start 161.75 124.618) (end 128.882 124.618) (width 0.254) (layer "B.Cu") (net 2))
 (segment (start 128.882 124.618) (end 123.37 130.13) (width 0.254) (layer "B.Cu") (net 2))
 (segment (start 129.809 123.5) (end 129.809 103.191) (width 0.254) (layer "F.Cu") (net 3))
 (segment (start 165.5 135.5) (end 165.5 133) (width 0.254) (layer "F.Cu") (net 3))
 (segment (start 129.81 138.5) (end 129.809 138.499) (width 0.254) (layer "F.Cu") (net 3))
 (segment (start 129.809 138.499) (end 129.809 124) (width 0.254) (layer "F.Cu") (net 3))
 (segment (start 129.809 103.191) (end 135.05 97.95) (width 0.254) (layer "F.Cu") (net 3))
 (segment (start 159 138.5) (end 162 135.5) (width 0.254) (layer "F.Cu") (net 3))
 (segment (start 129.809 124) (end 129.809 123.5) (width 0.254) (layer "F.Cu") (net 3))
 (segment (start 135.05 97.95) (end 135.05 85.09) (width 0.254) (layer "F.Cu") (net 3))
 (segment (start 162 135.5) (end 165.5 135.5) (width 0.254) (layer "F.Cu") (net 3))
 (segment (start 155.19 138.5) (end 159 138.5) (width 0.254) (layer "F.Cu") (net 3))
 (segment (start 139.129 137.319) (end 140.31 138.5) (width 0.254) (layer "B.Cu") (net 3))
 (segment (start 140.31 138.5) (end 140.5 138.5) (width 0.254) (layer "B.Cu") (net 3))
 (segment (start 129.81 138.5) (end 130.991 137.319) (width 0.254) (layer "B.Cu") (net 3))
 (segment (start 149.819 139.681) (end 151 138.5) (width 0.254) (layer "B.Cu") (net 3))
 (segment (start 151 138.5) (end 155.19 138.5) (width 0.254) (layer "B.Cu") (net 3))
 (segment (start 141.681 139.681) (end 149.819 139.681) (width 0.254) (layer "B.Cu") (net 3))
 (segment (start 130.991 137.319) (end 139.129 137.319) (width 0.254) (layer "B.Cu") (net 3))
 (segment (start 140.5 138.5) (end 141.681 139.681) (width 0.254) (layer "B.Cu") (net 3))
 (segment (start 168.5 121) (end 168.5 122.38) (width 0.254) (layer "F.Cu") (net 7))
 (segment (start 168.5 122.38) (end 165.5 125.38) (width 0.254) (layer "F.Cu") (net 7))
 (segment (start 155.37 125.38) (end 150.29 130.46) (width 0.254) (layer "B.Cu") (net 7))
 (segment (start 165.5 125.38) (end 155.37 125.38) (width 0.254) (layer "B.Cu") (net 7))
 (segment (start 150.29 130.46) (end 150.29 133.35) (width 0.254) (layer "B.Cu") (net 7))
 (segment (start 131.509 139.681) (end 132.69 138.5) (width 0.254) (layer "F.Cu") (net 1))
 (segment (start 147.75 135.25) (end 147.75 133.35) (width 0.254) (layer "F.Cu") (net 1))
 (segment (start 132.69 138.5) (end 133.871 137.319) (width 0.254) (layer "F.Cu") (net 1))
 (segment (start 119.3 138.5) (end 120.481 139.681) (width 0.254) (layer "F.Cu") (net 1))
 (segment (start 120.481 139.681) (end 131.509 139.681) (width 0.254) (layer "F.Cu") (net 1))
 (segment (start 145.681 137.319) (end 147.75 135.25) (width 0.254) (layer "F.Cu") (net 1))
 (segment (start 133.871 137.319) (end 145.681 137.319) (width 0.254) (layer "F.Cu") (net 1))
 (segment (start 154 136) (end 155.37 134.63) (width 0.254) (layer "F.Cu") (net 4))
 (segment (start 155.37 129.13) (end 155.37 133.35) (width 0.254) (layer "F.Cu") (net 4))
 (segment (start 149.5 136) (end 154 136) (width 0.254) (layer "F.Cu") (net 4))
 (segment (start 155.37 134.63) (end 155.37 133.35) (width 0.254) (layer "F.Cu") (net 4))
 (segment (start 143.38 138.5) (end 147 138.5) (width 0.254) (layer "F.Cu") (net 4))
 (segment (start 167.5 117) (end 155.37 129.13) (width 0.254) (layer "F.Cu") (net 4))
 (segment (start 147 138.5) (end 149.5 136) (width 0.254) (layer "F.Cu") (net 4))
 (segment (start 125.44 135.25) (end 126.5 135.25) (width 0.254) (layer "F.Cu") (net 6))
 (segment (start 145.21 130.94) (end 145.21 133.35) (width 0.254) (layer "F.Cu") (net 6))
 (segment (start 122.19 138.5) (end 125.44 135.25) (width 0.254) (layer "F.Cu") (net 6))
 (segment (start 167.65 108.5) (end 145.21 130.94) (width 0.254) (layer "F.Cu") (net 6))
 (via (at 126.5 135.25) (size 0.762) (drill 0.381) (layers "F.Cu" "B.Cu") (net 6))
 (segment (start 126.5 135.25) (end 143.31 135.25) (width 0.254) (layer "B.Cu") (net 6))
 (segment (start 143.31 135.25) (end 145.21 133.35) (width 0.254) (layer "B.Cu") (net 6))
 (segment (start 164.844 115.656) (end 164.844 118.877952) (width 0.254) (layer "F.Cu") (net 5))
 (segment (start 164.844 118.877952) (end 152.83 130.891952) (width 0.254) (layer "F.Cu") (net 5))
 (segment (start 152.83 130.891952) (end 152.83 133.35) (width 0.254) (layer "F.Cu") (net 5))
 (segment (start 167.5 113) (end 164.844 115.656) (width 0.254) (layer "F.Cu") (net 5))
 (segment (start 153 136) (end 152.83 135.83) (width 0.254) (layer "B.Cu") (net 5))
 (segment (start 160.5 138.5) (end 158 136) (width 0.254) (layer "B.Cu") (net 5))
 (segment (start 162.81 138.5) (end 160.5 138.5) (width 0.254) (layer "B.Cu") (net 5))
 (segment (start 152.83 135.83) (end 152.83 133.35) (width 0.254) (layer "B.Cu") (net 5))
 (segment (start 158 136) (end 153 136) (width 0.254) (layer "B.Cu") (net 5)))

